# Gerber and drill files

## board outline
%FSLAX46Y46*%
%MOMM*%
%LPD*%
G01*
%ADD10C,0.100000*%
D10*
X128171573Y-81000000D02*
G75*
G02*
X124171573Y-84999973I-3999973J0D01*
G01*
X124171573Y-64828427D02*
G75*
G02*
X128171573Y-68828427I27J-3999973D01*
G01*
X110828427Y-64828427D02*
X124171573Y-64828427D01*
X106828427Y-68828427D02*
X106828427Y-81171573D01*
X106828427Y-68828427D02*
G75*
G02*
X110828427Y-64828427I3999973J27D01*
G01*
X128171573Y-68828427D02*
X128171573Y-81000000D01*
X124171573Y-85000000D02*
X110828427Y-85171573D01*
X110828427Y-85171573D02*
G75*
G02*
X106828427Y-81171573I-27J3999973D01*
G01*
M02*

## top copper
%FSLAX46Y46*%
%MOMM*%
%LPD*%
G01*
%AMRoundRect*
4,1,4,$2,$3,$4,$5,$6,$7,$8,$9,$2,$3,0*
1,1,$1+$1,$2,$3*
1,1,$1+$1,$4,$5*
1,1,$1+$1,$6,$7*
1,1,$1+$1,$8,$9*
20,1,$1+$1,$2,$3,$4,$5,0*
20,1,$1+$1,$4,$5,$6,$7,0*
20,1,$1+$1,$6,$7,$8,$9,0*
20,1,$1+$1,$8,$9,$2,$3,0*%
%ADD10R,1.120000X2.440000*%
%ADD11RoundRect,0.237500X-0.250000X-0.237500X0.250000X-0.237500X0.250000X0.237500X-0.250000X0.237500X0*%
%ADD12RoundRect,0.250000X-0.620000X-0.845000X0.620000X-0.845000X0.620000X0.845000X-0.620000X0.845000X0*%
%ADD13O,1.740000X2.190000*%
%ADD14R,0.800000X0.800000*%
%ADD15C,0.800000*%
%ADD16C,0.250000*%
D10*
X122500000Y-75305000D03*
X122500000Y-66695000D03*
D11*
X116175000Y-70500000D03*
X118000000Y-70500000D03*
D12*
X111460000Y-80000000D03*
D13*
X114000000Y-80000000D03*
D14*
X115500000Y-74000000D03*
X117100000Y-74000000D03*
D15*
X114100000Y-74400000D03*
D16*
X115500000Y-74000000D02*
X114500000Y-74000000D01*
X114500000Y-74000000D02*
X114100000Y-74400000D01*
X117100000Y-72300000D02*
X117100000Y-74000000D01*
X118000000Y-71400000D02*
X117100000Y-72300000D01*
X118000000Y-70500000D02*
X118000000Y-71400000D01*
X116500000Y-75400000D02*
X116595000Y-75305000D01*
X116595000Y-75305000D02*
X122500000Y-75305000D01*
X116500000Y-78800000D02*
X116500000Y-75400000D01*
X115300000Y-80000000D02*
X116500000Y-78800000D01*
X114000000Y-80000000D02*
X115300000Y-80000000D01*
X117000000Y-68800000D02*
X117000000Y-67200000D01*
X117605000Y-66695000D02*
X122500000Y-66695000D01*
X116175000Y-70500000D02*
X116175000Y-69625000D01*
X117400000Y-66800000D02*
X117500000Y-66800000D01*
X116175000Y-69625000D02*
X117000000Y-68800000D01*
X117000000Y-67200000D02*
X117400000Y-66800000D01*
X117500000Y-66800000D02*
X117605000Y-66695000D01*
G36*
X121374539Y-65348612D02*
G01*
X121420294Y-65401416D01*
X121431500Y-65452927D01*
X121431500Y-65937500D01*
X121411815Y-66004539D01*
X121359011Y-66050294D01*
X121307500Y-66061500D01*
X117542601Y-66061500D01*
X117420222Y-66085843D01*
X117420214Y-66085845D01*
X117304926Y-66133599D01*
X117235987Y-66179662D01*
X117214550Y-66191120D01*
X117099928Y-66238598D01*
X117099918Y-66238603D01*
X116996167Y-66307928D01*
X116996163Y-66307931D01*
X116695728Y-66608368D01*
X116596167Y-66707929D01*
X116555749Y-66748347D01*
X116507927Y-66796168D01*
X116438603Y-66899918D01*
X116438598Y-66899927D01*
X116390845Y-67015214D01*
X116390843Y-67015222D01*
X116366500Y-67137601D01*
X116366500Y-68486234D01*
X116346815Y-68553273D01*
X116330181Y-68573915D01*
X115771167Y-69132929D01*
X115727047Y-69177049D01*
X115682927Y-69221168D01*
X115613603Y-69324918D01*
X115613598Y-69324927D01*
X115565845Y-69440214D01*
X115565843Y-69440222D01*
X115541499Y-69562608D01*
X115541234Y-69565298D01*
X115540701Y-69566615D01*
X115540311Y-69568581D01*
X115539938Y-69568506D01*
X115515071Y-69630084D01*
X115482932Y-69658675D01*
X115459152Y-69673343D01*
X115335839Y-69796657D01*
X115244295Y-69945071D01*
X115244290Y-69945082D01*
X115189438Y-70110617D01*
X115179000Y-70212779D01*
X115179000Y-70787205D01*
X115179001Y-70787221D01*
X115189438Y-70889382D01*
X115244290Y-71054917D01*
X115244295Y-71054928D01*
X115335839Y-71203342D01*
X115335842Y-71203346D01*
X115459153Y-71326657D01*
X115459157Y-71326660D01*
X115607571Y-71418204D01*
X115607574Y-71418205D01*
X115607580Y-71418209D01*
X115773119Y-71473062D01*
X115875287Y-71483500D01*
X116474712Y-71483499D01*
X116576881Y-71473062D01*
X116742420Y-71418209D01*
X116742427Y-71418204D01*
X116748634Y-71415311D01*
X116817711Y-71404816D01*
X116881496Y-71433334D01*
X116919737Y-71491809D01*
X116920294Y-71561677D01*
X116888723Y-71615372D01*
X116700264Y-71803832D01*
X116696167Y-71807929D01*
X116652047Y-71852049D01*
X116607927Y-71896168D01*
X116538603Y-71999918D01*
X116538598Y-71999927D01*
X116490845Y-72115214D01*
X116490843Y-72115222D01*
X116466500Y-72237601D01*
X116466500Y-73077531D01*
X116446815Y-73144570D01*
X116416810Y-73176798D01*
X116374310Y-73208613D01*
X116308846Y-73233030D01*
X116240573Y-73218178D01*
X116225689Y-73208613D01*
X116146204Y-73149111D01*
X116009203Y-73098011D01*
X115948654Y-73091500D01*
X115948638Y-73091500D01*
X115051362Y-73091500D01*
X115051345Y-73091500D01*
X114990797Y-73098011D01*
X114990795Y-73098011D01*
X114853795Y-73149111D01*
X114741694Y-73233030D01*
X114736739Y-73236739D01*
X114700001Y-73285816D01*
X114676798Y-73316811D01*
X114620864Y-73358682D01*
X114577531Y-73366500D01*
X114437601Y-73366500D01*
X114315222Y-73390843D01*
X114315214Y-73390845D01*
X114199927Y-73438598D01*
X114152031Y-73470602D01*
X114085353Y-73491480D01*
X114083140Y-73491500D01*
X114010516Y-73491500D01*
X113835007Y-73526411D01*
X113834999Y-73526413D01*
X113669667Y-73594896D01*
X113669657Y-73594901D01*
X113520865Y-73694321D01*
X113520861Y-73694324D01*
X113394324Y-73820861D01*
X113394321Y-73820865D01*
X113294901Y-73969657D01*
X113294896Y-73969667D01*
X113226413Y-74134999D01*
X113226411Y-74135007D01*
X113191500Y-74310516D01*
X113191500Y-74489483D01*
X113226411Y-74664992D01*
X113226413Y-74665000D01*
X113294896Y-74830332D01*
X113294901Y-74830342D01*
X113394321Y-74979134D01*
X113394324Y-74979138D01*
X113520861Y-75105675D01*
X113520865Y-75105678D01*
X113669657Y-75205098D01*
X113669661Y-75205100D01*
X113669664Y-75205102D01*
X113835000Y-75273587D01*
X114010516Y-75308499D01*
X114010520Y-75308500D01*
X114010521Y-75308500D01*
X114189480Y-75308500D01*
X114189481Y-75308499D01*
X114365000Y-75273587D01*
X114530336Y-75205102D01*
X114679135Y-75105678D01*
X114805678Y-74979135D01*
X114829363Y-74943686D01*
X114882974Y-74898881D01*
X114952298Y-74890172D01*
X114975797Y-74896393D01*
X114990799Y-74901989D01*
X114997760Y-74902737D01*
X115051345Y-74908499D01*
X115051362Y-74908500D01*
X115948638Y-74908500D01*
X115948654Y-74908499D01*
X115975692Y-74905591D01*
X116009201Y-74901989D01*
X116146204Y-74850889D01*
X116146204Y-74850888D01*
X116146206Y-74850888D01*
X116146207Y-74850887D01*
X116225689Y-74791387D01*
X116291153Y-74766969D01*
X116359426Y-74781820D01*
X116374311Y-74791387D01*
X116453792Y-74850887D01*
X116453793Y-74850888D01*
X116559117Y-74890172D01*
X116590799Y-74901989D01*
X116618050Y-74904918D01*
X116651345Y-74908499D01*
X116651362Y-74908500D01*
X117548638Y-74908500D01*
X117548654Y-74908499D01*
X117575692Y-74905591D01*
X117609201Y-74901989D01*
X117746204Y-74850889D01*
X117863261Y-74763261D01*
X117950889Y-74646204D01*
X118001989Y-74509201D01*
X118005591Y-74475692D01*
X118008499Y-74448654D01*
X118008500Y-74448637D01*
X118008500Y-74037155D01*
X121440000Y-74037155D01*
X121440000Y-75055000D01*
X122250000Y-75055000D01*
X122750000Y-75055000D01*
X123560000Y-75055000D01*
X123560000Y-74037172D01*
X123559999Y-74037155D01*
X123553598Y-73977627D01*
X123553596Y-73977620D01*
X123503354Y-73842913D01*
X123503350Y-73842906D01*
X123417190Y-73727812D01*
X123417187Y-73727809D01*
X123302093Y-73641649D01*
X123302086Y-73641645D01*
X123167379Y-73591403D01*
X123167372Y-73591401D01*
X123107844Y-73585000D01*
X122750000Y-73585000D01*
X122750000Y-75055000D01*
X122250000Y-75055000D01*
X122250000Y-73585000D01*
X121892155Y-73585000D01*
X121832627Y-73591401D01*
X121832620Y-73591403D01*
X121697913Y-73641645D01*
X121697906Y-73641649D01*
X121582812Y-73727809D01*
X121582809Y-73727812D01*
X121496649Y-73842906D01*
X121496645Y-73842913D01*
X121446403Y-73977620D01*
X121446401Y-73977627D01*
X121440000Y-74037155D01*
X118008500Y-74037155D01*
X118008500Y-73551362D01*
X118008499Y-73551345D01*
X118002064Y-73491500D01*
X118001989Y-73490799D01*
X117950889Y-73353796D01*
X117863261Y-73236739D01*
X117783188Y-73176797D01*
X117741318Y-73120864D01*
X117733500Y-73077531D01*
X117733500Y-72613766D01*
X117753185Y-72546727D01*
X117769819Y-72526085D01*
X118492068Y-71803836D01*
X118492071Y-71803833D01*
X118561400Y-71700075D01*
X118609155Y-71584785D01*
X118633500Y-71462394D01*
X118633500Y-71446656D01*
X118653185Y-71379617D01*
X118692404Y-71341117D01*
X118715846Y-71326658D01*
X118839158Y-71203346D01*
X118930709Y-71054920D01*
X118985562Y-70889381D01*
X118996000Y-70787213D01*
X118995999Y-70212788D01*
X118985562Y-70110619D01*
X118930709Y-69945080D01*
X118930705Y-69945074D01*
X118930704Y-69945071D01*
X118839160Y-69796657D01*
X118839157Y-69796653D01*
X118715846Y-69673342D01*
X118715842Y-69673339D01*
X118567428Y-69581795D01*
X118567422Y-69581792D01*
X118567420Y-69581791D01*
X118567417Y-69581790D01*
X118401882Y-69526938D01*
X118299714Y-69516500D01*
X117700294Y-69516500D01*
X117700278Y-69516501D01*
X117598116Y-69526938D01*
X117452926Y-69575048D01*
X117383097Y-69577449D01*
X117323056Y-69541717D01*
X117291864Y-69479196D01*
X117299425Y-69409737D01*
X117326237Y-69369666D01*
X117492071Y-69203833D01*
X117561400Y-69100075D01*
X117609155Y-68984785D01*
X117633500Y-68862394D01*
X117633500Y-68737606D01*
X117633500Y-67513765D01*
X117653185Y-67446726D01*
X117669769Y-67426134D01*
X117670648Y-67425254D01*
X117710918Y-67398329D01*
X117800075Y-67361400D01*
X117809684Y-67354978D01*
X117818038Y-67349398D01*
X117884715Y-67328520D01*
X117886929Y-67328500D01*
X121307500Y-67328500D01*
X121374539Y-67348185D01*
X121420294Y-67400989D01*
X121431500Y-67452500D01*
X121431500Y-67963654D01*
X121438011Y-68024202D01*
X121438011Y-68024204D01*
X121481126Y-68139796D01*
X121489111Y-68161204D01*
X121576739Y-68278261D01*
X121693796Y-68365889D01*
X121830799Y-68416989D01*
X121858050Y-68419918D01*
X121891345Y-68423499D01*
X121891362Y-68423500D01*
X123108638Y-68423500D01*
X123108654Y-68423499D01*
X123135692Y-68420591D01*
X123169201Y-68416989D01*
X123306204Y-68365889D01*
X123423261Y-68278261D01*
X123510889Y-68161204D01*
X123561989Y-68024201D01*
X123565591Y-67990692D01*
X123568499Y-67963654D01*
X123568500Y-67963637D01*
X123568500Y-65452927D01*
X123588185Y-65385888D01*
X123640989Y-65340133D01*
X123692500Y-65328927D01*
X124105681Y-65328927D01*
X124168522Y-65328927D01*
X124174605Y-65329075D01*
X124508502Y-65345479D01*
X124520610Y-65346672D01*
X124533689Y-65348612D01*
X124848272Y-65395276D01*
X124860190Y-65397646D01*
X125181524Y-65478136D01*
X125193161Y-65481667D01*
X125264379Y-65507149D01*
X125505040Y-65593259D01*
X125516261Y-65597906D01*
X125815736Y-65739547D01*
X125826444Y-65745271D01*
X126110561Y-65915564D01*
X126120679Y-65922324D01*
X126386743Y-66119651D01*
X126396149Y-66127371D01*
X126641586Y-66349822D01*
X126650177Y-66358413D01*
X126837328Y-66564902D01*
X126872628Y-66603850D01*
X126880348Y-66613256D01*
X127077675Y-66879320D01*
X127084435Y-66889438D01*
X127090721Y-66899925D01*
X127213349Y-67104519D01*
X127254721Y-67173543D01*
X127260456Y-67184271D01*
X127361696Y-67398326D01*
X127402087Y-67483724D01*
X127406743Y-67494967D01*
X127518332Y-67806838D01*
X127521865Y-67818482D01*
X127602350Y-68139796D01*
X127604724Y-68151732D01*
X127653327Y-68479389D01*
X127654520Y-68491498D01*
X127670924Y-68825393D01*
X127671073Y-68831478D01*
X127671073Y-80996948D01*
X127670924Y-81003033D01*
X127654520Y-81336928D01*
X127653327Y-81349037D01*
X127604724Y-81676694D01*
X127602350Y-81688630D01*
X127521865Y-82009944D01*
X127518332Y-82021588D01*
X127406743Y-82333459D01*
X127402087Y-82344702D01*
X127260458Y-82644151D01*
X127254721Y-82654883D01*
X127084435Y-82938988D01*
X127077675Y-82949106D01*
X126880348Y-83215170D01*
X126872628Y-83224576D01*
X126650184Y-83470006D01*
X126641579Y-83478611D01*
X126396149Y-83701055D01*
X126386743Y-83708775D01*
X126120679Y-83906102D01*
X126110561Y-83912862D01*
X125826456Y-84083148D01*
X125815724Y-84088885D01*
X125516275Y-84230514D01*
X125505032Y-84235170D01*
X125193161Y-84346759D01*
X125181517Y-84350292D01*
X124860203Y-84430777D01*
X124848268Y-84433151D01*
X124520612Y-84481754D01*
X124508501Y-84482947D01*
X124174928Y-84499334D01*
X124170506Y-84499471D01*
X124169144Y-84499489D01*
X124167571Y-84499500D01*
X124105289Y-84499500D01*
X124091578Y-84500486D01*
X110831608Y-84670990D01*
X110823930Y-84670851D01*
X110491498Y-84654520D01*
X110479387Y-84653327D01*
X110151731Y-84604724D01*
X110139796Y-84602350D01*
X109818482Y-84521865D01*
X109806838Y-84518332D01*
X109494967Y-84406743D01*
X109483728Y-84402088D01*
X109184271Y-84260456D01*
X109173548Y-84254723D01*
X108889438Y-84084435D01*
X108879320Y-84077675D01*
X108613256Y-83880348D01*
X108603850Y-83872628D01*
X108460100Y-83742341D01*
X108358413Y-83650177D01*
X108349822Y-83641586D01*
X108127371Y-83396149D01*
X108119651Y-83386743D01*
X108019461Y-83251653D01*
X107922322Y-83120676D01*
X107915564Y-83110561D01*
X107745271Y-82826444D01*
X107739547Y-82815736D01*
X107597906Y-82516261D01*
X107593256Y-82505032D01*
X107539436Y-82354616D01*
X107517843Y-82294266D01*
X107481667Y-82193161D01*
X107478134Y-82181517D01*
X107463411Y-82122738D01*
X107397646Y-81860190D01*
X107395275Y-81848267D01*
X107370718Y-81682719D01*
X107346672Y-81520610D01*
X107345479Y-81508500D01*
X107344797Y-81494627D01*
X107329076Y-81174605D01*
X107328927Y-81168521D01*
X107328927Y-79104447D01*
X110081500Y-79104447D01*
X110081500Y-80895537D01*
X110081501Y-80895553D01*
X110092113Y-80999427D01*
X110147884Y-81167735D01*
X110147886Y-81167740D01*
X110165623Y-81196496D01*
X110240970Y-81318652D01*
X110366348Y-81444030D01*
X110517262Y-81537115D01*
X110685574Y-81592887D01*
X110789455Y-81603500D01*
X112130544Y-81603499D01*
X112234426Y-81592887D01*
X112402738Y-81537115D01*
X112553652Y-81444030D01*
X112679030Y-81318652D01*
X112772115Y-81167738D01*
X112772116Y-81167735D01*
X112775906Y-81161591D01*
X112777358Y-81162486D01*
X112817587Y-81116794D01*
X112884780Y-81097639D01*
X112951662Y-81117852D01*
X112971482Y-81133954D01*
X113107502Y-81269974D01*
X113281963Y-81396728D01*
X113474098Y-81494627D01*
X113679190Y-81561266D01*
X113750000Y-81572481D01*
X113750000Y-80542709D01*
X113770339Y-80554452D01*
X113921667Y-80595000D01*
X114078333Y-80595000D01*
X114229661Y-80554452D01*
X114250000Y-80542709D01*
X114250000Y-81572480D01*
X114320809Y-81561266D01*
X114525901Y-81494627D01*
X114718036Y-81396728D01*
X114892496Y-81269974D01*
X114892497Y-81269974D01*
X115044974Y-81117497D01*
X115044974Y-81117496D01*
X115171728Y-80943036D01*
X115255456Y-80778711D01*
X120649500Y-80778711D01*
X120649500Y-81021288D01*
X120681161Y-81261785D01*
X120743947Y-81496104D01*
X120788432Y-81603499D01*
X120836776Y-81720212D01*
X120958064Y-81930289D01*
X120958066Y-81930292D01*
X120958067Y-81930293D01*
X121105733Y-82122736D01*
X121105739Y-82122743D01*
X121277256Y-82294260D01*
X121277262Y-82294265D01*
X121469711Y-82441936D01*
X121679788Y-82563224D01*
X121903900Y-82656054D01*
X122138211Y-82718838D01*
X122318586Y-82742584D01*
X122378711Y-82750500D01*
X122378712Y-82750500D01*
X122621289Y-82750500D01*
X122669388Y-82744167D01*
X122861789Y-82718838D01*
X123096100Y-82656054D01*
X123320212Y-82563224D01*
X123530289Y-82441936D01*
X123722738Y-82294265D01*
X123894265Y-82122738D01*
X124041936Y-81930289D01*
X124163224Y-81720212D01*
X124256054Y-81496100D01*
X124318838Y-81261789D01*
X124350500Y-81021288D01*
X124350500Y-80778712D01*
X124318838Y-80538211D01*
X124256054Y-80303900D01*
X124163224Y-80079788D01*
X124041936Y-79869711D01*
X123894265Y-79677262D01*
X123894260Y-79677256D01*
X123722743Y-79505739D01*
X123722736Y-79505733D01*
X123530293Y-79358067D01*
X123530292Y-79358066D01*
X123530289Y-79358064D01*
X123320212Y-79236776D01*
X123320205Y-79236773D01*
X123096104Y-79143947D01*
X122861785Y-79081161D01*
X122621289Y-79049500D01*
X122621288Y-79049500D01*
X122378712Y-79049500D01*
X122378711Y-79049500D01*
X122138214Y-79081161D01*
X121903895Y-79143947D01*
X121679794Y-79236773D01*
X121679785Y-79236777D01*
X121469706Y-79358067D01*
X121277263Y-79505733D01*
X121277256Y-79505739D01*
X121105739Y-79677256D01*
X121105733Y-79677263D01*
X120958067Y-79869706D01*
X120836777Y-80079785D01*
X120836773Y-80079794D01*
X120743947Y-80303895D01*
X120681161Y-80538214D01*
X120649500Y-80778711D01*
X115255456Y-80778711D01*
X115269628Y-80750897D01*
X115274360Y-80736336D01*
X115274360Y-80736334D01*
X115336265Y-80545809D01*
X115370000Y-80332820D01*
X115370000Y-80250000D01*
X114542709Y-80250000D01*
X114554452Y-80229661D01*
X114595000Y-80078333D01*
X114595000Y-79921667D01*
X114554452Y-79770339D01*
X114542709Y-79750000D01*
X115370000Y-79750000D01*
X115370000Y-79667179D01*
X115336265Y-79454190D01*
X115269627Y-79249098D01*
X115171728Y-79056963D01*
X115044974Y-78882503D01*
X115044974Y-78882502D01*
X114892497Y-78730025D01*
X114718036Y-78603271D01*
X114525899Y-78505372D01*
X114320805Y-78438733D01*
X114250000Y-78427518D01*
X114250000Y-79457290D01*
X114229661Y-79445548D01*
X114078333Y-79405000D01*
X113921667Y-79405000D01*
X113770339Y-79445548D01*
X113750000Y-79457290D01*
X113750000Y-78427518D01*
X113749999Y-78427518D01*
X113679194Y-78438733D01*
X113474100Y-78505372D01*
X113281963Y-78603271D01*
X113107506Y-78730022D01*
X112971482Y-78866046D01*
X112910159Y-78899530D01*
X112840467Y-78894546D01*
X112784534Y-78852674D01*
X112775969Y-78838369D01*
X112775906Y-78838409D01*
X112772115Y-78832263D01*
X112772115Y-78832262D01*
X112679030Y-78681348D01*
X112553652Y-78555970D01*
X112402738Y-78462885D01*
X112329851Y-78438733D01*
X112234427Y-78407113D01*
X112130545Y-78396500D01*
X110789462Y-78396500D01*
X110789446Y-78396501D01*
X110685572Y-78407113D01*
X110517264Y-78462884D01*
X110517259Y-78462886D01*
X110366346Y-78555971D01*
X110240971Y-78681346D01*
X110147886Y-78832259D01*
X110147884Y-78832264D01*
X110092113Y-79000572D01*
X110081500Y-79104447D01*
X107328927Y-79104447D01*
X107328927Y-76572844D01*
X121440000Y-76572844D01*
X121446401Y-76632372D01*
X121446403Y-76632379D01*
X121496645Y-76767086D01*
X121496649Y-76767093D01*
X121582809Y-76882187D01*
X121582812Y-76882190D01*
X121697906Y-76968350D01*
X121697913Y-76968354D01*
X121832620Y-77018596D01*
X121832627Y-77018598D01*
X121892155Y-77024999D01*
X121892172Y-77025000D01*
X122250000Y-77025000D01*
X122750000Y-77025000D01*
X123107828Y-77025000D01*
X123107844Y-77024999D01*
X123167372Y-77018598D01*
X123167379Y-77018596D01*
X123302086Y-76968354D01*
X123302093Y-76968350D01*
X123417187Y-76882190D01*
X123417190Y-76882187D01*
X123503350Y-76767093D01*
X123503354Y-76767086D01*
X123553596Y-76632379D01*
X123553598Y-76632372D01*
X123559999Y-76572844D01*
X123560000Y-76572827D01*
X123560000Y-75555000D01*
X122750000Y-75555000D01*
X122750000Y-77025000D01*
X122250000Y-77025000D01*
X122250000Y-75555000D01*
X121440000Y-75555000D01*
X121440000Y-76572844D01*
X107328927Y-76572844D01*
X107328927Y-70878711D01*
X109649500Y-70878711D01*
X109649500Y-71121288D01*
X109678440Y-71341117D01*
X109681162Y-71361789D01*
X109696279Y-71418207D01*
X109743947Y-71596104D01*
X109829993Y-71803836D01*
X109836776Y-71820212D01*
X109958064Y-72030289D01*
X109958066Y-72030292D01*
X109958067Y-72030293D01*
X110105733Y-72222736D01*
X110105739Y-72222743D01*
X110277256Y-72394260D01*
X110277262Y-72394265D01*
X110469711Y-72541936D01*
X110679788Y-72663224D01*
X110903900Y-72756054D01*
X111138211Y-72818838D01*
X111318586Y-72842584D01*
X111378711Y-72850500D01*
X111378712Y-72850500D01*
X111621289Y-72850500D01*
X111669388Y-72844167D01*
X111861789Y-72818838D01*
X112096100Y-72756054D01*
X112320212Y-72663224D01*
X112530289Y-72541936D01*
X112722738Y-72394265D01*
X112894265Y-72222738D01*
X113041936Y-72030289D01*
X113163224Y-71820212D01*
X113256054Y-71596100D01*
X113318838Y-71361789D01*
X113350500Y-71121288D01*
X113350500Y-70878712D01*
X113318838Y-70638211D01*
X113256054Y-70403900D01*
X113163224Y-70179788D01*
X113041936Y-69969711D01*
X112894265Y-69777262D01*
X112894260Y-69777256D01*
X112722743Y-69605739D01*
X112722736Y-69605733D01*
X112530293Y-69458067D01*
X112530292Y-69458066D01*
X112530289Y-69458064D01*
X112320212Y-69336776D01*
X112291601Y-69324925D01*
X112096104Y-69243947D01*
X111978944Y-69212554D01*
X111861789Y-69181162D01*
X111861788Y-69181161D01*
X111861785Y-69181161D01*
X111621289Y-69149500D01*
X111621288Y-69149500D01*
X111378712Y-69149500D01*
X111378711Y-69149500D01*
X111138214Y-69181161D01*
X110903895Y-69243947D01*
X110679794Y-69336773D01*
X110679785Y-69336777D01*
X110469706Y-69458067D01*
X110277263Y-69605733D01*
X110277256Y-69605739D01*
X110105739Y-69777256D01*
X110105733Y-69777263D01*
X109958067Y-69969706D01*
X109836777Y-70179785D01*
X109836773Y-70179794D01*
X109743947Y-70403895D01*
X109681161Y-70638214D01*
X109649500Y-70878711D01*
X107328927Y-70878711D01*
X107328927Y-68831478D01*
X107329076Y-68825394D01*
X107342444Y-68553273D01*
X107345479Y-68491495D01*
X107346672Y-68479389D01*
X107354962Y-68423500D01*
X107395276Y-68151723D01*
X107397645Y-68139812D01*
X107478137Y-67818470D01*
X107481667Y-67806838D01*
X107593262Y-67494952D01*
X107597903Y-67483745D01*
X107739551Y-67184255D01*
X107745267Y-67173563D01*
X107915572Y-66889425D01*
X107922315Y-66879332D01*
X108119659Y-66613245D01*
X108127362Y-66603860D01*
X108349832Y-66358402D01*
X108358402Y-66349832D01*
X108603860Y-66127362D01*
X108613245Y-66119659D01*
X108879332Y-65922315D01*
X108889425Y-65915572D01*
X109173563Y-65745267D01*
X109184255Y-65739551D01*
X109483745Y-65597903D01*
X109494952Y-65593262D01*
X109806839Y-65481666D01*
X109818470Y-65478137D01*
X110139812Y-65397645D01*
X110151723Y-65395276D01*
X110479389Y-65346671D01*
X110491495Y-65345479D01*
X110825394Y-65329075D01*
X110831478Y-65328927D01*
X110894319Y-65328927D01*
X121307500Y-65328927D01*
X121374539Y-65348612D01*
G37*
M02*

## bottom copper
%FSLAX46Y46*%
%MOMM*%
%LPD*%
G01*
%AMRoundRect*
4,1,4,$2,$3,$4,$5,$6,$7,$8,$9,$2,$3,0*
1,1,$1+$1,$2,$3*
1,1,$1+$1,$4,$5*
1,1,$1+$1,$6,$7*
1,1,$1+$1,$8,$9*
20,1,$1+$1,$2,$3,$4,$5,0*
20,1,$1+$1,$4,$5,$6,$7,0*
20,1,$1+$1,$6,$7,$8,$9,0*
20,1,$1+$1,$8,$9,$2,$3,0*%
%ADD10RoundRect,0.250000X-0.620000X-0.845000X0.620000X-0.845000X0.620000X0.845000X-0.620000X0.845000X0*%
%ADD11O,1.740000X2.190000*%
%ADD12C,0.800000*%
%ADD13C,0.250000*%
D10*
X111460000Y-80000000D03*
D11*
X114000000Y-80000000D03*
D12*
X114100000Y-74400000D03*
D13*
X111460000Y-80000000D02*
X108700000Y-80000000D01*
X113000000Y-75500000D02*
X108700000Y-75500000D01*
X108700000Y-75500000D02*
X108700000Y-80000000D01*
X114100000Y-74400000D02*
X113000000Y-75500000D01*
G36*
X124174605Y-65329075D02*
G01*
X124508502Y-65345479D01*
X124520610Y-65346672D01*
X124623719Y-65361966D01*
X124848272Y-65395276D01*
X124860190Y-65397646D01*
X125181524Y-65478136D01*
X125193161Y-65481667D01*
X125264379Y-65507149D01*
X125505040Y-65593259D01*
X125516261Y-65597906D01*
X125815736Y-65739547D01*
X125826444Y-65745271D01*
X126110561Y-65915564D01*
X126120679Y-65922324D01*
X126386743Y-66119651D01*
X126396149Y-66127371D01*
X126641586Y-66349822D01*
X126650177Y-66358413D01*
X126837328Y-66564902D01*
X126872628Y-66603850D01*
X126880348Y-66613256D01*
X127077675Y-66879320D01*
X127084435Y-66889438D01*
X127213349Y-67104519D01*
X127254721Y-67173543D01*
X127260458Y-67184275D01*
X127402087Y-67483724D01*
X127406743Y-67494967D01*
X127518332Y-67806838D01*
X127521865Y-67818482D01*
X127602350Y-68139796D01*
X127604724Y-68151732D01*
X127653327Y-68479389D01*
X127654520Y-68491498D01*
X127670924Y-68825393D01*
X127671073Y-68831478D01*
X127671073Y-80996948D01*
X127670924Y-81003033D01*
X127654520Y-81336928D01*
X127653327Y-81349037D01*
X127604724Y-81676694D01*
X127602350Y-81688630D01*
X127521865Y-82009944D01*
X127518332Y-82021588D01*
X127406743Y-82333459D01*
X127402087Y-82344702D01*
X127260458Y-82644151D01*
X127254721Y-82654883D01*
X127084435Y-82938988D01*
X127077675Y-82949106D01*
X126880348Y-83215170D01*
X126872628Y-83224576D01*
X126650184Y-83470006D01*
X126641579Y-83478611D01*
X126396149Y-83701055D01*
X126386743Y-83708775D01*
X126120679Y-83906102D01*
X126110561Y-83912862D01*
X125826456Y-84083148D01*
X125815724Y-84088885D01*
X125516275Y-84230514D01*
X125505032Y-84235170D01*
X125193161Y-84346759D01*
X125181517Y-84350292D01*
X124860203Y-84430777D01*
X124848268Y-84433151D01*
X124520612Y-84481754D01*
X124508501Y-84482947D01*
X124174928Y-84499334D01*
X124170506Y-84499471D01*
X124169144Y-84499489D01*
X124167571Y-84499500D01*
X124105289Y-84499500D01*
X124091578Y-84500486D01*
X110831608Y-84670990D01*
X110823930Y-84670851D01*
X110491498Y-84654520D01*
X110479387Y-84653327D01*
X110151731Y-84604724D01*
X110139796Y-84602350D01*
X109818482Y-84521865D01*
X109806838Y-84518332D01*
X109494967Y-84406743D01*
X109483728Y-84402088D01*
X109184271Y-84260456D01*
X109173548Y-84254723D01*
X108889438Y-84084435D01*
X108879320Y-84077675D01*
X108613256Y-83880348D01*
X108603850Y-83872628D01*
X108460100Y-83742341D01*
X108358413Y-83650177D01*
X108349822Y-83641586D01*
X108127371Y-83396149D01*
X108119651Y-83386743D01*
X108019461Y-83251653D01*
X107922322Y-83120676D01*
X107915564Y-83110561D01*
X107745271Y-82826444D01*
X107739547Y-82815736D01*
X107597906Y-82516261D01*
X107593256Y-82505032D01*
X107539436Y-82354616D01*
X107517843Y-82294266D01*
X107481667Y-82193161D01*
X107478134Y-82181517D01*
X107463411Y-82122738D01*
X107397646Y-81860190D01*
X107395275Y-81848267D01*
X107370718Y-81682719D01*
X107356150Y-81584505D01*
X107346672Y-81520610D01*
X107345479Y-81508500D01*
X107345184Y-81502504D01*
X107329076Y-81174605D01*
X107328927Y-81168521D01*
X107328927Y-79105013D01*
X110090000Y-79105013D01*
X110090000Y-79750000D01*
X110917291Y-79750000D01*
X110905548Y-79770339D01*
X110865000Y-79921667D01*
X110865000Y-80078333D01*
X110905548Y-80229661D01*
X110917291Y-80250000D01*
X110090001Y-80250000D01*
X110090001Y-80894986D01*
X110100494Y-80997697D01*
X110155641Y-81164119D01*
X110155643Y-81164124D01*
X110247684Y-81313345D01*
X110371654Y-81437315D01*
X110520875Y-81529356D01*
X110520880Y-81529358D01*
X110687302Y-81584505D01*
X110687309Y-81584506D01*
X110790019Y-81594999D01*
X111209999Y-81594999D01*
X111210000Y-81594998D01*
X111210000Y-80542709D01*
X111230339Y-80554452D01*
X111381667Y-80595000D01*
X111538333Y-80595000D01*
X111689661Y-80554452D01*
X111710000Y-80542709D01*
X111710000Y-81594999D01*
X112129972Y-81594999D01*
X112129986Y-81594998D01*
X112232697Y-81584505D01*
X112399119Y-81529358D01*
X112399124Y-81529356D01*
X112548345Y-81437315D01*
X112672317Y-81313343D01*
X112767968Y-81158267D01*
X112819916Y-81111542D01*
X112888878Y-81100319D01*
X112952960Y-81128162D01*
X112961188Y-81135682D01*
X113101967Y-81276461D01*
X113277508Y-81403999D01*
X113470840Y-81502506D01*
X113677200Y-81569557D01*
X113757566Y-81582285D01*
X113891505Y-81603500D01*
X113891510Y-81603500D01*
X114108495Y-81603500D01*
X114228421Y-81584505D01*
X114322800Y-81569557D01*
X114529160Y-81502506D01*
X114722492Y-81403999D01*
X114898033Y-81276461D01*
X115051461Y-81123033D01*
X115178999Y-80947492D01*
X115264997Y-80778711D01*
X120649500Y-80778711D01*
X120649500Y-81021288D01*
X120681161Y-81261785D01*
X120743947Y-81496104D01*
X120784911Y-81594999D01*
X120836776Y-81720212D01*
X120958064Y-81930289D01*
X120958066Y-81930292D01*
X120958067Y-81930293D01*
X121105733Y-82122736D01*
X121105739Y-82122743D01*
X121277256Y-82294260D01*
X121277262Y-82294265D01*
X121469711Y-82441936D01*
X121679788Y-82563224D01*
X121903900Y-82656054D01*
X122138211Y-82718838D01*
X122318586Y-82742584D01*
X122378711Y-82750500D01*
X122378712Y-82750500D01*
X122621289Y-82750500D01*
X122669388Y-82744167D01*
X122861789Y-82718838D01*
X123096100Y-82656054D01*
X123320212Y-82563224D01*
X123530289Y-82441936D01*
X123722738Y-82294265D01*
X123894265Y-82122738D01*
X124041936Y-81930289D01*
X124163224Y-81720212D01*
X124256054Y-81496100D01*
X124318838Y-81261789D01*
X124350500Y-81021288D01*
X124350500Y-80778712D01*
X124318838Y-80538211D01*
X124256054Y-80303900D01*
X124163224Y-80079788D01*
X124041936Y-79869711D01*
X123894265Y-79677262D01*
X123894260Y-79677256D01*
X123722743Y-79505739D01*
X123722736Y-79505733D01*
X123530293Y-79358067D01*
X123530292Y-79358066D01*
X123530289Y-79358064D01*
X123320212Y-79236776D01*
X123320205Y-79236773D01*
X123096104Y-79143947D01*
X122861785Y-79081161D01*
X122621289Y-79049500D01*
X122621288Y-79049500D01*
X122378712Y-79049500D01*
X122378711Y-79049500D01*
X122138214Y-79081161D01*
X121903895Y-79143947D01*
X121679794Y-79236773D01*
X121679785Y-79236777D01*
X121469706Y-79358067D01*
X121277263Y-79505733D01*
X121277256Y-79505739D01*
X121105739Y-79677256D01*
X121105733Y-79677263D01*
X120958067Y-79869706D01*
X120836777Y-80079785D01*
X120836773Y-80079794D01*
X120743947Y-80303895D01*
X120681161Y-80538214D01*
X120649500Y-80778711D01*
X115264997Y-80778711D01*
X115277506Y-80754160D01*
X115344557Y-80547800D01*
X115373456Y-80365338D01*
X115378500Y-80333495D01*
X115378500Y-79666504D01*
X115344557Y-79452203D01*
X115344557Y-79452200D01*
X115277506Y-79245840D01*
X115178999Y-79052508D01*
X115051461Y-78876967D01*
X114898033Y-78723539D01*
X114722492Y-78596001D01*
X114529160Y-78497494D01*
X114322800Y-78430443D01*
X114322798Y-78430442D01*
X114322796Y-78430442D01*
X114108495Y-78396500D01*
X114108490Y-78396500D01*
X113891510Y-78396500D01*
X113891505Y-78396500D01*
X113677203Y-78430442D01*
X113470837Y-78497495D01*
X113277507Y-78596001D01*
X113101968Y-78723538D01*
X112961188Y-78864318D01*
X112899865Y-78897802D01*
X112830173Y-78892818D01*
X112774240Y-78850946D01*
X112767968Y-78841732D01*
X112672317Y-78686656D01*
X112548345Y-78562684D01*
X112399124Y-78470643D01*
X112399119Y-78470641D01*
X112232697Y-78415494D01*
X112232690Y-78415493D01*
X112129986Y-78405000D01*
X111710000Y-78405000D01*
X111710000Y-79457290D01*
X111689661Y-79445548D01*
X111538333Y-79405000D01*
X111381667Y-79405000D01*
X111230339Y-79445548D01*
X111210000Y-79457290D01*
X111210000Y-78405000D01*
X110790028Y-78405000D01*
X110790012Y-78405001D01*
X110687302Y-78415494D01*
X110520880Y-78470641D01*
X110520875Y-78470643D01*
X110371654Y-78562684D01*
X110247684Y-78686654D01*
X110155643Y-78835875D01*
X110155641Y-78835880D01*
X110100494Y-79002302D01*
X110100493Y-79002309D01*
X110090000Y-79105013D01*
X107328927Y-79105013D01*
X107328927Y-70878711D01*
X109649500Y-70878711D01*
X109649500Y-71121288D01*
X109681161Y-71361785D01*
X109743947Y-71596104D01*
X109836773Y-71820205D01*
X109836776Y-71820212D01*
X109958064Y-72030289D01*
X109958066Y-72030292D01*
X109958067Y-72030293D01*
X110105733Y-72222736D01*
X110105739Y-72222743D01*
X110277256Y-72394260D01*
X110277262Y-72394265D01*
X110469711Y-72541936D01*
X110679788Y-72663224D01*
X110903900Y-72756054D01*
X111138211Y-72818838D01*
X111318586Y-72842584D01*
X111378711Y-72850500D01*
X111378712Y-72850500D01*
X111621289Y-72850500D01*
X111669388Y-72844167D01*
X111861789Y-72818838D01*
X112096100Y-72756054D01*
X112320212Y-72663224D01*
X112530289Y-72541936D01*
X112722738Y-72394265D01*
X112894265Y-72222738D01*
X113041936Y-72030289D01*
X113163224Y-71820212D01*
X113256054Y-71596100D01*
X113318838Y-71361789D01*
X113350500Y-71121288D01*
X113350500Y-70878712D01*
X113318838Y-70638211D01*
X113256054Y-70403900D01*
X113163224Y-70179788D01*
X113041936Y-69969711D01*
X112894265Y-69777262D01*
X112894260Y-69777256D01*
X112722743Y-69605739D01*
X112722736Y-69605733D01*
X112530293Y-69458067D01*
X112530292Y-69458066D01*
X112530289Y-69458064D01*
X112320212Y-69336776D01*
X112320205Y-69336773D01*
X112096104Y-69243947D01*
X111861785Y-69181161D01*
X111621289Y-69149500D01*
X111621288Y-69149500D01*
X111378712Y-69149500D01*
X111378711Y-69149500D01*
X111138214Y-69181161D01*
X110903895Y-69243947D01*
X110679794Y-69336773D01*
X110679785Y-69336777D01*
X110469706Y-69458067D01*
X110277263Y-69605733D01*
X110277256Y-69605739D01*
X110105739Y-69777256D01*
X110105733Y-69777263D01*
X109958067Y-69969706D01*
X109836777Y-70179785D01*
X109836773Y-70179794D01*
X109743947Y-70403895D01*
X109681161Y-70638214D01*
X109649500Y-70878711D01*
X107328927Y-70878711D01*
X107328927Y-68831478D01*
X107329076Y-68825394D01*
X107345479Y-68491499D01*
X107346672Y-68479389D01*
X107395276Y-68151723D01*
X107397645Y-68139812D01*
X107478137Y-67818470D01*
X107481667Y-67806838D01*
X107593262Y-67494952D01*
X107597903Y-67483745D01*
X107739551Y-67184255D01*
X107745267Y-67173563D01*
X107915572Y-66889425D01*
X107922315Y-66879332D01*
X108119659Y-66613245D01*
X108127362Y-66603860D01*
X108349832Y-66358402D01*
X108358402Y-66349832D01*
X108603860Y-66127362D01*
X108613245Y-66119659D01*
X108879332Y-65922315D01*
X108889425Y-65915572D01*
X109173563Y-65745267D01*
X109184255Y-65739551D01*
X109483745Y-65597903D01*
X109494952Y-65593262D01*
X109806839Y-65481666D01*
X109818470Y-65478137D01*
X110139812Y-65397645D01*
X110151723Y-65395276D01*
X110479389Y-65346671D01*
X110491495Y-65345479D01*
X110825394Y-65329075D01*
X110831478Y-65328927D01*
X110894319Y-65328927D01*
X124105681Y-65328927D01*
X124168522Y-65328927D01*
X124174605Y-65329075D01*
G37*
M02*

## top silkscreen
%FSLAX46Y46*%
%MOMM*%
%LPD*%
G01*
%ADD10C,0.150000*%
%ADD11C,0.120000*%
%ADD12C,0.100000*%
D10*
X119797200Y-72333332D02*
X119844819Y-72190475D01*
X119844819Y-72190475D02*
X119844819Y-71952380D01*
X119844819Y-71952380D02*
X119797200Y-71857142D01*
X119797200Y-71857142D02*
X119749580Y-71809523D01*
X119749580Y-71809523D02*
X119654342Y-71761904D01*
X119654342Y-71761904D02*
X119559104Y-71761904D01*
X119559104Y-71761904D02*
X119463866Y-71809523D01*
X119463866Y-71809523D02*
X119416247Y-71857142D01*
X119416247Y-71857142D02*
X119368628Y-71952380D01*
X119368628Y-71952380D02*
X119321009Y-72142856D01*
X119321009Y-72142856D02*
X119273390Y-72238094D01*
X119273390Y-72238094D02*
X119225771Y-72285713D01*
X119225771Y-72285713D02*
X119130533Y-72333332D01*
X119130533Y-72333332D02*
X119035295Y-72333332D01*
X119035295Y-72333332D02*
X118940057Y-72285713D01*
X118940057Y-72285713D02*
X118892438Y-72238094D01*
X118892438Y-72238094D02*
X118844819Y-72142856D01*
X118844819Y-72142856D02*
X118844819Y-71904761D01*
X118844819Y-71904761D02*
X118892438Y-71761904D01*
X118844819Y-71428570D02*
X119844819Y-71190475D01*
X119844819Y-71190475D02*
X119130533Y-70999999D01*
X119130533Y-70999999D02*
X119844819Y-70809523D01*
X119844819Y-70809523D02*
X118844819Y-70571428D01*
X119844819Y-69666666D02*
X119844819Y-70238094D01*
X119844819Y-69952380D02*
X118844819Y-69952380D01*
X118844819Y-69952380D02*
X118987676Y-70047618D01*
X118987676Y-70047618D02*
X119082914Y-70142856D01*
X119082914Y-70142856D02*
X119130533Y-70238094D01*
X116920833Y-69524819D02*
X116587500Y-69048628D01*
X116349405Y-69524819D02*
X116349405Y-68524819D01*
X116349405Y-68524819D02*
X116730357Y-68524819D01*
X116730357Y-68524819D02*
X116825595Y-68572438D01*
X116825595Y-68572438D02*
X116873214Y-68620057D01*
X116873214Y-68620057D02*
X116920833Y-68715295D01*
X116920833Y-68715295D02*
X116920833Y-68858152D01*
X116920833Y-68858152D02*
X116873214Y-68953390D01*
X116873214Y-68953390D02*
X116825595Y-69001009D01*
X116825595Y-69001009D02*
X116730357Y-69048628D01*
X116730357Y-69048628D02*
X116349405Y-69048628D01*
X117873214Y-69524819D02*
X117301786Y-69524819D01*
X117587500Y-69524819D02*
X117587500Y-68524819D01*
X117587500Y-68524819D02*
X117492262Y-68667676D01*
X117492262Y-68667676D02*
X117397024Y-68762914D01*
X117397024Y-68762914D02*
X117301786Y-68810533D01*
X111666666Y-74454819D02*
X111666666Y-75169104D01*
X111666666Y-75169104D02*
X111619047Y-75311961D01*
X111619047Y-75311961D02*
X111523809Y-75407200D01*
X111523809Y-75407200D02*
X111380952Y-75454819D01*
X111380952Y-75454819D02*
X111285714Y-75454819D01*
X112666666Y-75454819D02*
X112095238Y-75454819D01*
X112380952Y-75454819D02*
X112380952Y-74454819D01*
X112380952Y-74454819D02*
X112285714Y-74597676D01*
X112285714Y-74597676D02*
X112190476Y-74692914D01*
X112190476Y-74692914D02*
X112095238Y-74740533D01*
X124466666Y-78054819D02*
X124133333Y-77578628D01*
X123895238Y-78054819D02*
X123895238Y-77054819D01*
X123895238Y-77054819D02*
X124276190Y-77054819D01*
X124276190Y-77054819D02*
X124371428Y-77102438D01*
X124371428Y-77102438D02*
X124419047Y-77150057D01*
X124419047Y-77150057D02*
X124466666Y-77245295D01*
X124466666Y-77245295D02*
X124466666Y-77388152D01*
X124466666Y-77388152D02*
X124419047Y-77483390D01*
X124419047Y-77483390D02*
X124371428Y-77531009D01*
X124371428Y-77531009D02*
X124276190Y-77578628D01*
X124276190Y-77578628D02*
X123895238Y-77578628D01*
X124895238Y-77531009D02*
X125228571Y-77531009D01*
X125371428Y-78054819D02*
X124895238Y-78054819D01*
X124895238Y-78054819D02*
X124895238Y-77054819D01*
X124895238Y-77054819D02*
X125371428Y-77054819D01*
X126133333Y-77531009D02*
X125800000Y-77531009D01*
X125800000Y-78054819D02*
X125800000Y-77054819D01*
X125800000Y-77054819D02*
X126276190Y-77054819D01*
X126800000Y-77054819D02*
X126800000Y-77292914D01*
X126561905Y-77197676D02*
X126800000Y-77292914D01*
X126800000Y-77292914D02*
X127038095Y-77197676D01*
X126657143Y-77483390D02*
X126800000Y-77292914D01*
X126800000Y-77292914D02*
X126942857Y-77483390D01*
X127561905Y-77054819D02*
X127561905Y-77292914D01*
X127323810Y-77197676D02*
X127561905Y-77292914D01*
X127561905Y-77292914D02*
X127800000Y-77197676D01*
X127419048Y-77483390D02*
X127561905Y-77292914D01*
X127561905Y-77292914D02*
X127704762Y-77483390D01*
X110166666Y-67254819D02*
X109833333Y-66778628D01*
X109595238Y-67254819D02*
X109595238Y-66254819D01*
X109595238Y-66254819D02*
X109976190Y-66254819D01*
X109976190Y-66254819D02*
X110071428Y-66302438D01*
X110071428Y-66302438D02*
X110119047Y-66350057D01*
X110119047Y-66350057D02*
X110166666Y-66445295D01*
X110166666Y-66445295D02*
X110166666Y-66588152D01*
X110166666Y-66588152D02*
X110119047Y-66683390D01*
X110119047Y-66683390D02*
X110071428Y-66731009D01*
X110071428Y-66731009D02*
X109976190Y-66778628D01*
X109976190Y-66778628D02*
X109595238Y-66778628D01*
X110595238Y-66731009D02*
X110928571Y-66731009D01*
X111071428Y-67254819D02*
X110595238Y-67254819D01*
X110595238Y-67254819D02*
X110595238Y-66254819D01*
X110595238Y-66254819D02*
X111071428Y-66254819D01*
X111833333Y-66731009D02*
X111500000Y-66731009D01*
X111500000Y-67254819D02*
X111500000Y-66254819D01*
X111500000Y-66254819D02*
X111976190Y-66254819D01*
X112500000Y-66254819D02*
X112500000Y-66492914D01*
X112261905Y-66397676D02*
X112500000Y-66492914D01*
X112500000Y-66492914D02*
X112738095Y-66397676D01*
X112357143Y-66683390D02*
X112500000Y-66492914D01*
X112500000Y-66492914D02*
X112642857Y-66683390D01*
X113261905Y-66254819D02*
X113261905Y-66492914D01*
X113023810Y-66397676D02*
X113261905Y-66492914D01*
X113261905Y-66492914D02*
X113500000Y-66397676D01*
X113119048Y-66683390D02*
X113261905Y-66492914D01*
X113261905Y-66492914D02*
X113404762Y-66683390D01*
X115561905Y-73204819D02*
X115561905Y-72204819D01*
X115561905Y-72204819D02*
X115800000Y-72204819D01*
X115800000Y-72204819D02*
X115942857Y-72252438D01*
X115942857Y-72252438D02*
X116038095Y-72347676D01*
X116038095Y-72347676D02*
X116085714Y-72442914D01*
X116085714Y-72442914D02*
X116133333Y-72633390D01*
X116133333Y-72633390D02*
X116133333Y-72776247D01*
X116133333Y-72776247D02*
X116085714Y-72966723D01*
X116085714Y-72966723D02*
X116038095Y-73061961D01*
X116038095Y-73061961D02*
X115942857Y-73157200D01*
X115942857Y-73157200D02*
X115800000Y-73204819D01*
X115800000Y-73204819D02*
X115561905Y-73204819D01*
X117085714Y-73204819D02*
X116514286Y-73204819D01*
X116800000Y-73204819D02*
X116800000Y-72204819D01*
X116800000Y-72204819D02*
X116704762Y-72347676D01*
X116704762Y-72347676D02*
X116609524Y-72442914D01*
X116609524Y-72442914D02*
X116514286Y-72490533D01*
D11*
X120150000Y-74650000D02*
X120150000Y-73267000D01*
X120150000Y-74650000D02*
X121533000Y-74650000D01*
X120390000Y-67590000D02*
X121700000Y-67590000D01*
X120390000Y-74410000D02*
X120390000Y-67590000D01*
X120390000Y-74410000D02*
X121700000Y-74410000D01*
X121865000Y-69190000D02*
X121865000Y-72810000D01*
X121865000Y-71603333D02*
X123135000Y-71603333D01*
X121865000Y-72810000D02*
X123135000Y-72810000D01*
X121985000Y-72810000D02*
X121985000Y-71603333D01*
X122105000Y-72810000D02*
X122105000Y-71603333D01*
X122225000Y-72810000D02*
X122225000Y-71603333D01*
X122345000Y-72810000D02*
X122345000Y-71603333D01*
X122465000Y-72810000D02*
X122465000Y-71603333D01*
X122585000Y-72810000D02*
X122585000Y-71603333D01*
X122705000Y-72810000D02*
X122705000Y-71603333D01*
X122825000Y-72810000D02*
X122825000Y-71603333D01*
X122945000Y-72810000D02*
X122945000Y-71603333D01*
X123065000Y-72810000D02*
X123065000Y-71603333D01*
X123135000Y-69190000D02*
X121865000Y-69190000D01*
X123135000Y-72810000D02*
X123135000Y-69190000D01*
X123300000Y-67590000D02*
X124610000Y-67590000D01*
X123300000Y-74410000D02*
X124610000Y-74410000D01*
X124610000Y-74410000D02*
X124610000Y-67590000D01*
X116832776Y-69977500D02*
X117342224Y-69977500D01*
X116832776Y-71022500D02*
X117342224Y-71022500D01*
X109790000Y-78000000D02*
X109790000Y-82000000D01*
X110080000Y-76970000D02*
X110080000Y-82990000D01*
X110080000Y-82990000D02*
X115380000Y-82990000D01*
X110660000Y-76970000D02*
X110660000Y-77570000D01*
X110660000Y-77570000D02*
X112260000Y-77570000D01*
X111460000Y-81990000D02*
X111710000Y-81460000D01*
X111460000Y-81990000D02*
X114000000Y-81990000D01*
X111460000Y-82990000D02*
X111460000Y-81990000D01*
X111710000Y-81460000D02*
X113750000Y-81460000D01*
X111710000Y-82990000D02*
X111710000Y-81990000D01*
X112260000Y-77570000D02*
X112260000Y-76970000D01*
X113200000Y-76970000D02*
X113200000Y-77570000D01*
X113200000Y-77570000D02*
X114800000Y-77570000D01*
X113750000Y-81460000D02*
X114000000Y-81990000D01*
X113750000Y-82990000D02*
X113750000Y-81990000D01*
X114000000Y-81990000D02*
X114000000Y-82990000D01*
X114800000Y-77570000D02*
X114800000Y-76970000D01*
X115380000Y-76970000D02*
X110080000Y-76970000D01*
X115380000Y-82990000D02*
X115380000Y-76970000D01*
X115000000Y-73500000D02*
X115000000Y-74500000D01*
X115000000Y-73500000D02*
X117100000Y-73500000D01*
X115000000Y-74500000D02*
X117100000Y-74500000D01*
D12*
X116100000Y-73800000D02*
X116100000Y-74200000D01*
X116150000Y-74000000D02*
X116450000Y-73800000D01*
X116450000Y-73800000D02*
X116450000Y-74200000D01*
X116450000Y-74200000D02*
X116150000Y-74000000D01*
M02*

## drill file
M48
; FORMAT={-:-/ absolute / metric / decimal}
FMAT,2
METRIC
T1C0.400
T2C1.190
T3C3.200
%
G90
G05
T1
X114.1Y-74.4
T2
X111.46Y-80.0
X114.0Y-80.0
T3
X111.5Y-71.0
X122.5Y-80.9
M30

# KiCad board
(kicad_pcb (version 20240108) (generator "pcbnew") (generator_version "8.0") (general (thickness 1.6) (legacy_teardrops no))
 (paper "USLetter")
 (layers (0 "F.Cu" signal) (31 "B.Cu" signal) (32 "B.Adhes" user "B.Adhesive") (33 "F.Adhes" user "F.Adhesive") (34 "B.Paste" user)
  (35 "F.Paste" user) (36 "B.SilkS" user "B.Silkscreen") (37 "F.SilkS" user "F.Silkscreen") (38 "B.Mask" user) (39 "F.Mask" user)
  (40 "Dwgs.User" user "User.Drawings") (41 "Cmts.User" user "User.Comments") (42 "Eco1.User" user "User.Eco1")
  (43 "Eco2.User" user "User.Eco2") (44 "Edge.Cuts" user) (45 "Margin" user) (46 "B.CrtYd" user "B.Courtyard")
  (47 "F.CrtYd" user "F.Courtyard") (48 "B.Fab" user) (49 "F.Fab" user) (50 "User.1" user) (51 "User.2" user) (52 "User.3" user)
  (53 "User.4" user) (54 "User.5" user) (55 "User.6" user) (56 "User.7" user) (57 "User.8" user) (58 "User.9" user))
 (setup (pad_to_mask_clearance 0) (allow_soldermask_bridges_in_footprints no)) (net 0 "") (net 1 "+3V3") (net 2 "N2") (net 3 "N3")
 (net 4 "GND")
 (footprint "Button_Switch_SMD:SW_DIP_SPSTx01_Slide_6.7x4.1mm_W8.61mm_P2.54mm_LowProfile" (layer "F.Cu") (at 122.5 71 90)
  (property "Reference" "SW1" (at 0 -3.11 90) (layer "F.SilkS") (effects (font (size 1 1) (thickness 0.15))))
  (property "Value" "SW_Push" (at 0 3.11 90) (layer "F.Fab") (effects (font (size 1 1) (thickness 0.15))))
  (fp_line (start -3.65 -2.35) (end -2.267 -2.35) (stroke (width 0.12) (type solid)) (layer "F.SilkS"))
  (fp_line (start -3.65 -2.35) (end -3.65 -0.967) (stroke (width 0.12) (type solid)) (layer "F.SilkS"))
  (fp_line (start 3.41 -2.11) (end 3.41 -0.8) (stroke (width 0.12) (type solid)) (layer "F.SilkS"))
  (fp_line (start -3.41 -2.11) (end 3.41 -2.11) (stroke (width 0.12) (type solid)) (layer "F.SilkS"))
  (fp_line (start -3.41 -2.11) (end -3.41 -0.8) (stroke (width 0.12) (type solid)) (layer "F.SilkS"))
  (fp_line (start 1.81 -0.635) (end -1.81 -0.635) (stroke (width 0.12) (type solid)) (layer "F.SilkS"))
  (fp_line (start -0.603333 -0.635) (end -0.603333 0.635) (stroke (width 0.12) (type solid)) (layer "F.SilkS"))
  (fp_line (start -1.81 -0.635) (end -1.81 0.635) (stroke (width 0.12) (type solid)) (layer "F.SilkS"))
  (fp_line (start -1.81 -0.515) (end -0.603333 -0.515) (stroke (width 0.12) (type solid)) (layer "F.SilkS"))
  (fp_line (start -1.81 -0.395) (end -0.603333 -0.395) (stroke (width 0.12) (type solid)) (layer "F.SilkS"))
  (fp_line (start -1.81 -0.275) (end -0.603333 -0.275) (stroke (width 0.12) (type solid)) (layer "F.SilkS"))
  (fp_line (start -1.81 -0.155) (end -0.603333 -0.155) (stroke (width 0.12) (type solid)) (layer "F.SilkS"))
  (fp_line (start -1.81 -0.035) (end -0.603333 -0.035) (stroke (width 0.12) (type solid)) (layer "F.SilkS"))
  (fp_line (start -1.81 0.085) (end -0.603333 0.085) (stroke (width 0.12) (type solid)) (layer "F.SilkS"))
  (fp_line (start -1.81 0.205) (end -0.603333 0.205) (stroke (width 0.12) (type solid)) (layer "F.SilkS"))
  (fp_line (start -1.81 0.325) (end -0.603333 0.325) (stroke (width 0.12) (type solid)) (layer "F.SilkS"))
  (fp_line (start -1.81 0.445) (end -0.603333 0.445) (stroke (width 0.12) (type solid)) (layer "F.SilkS"))
  (fp_line (start -1.81 0.565) (end -0.603333 0.565) (stroke (width 0.12) (type solid)) (layer "F.SilkS"))
  (fp_line (start 1.81 0.635) (end 1.81 -0.635) (stroke (width 0.12) (type solid)) (layer "F.SilkS"))
  (fp_line (start -1.81 0.635) (end 1.81 0.635) (stroke (width 0.12) (type solid)) (layer "F.SilkS"))
  (fp_line (start 3.41 0.8) (end 3.41 2.11) (stroke (width 0.12) (type solid)) (layer "F.SilkS"))
  (fp_line (start -3.41 0.8) (end -3.41 2.11) (stroke (width 0.12) (type solid)) (layer "F.SilkS"))
  (fp_line (start -3.41 2.11) (end 3.41 2.11) (stroke (width 0.12) (type solid)) (layer "F.SilkS"))
  (pad "1" smd rect (at -4.305 0 90) (size 2.44 1.12) (layers "F.Cu" "F.Paste" "F.Mask") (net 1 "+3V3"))
  (pad "2" smd rect (at 4.305 0 90) (size 2.44 1.12) (layers "F.Cu" "F.Paste" "F.Mask") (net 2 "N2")))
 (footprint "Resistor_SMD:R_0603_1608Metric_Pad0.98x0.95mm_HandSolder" (layer "F.Cu") (at 117.0875 70.5)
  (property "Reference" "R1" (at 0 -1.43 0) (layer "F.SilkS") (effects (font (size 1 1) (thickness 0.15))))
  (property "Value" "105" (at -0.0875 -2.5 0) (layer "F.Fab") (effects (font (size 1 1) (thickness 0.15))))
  (fp_line (start -0.254724 -0.5225) (end 0.254724 -0.5225) (stroke (width 0.12) (type solid)) (layer "F.SilkS"))
  (fp_line (start -0.254724 0.5225) (end 0.254724 0.5225) (stroke (width 0.12) (type solid)) (layer "F.SilkS"))
  (pad "1" smd roundrect (at -0.9125 0) (size 0.975 0.95) (layers "F.Cu" "F.Paste" "F.Mask") (roundrect_rratio 0.25) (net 2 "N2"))
  (pad "2" smd roundrect (at 0.9125 0) (size 0.975 0.95) (layers "F.Cu" "F.Paste" "F.Mask") (roundrect_rratio 0.25) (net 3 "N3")))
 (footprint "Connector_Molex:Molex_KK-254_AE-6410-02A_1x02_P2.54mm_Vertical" (layer "F.Cu") (at 111.46 80)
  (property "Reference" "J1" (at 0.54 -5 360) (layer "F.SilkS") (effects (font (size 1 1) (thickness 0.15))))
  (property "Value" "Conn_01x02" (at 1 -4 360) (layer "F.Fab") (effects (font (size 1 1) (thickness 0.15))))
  (fp_line (start -1.67 -2) (end -1.67 2) (stroke (width 0.12) (type solid)) (layer "F.SilkS"))
  (fp_line (start -1.38 -3.03) (end -1.38 2.99) (stroke (width 0.12) (type solid)) (layer "F.SilkS"))
  (fp_line (start -1.38 2.99) (end 3.92 2.99) (stroke (width 0.12) (type solid)) (layer "F.SilkS"))
  (fp_line (start -0.8 -3.03) (end -0.8 -2.43) (stroke (width 0.12) (type solid)) (layer "F.SilkS"))
  (fp_line (start -0.8 -2.43) (end 0.8 -2.43) (stroke (width 0.12) (type solid)) (layer "F.SilkS"))
  (fp_line (start 0 1.99) (end 0.25 1.46) (stroke (width 0.12) (type solid)) (layer "F.SilkS"))
  (fp_line (start 0 1.99) (end 2.54 1.99) (stroke (width 0.12) (type solid)) (layer "F.SilkS"))
  (fp_line (start 0 2.99) (end 0 1.99) (stroke (width 0.12) (type solid)) (layer "F.SilkS"))
  (fp_line (start 0.25 1.46) (end 2.29 1.46) (stroke (width 0.12) (type solid)) (layer "F.SilkS"))
  (fp_line (start 0.25 2.99) (end 0.25 1.99) (stroke (width 0.12) (type solid)) (layer "F.SilkS"))
  (fp_line (start 0.8 -2.43) (end 0.8 -3.03) (stroke (width 0.12) (type solid)) (layer "F.SilkS"))
  (fp_line (start 1.74 -3.03) (end 1.74 -2.43) (stroke (width 0.12) (type solid)) (layer "F.SilkS"))
  (fp_line (start 1.74 -2.43) (end 3.34 -2.43) (stroke (width 0.12) (type solid)) (layer "F.SilkS"))
  (fp_line (start 2.29 1.46) (end 2.54 1.99) (stroke (width 0.12) (type solid)) (layer "F.SilkS"))
  (fp_line (start 2.29 2.99) (end 2.29 1.99) (stroke (width 0.12) (type solid)) (layer "F.SilkS"))
  (fp_line (start 2.54 1.99) (end 2.54 2.99) (stroke (width 0.12) (type solid)) (layer "F.SilkS"))
  (fp_line (start 3.34 -2.43) (end 3.34 -3.03) (stroke (width 0.12) (type solid)) (layer "F.SilkS"))
  (fp_line (start 3.92 -3.03) (end -1.38 -3.03) (stroke (width 0.12) (type solid)) (layer "F.SilkS"))
  (fp_line (start 3.92 2.99) (end 3.92 -3.03) (stroke (width 0.12) (type solid)) (layer "F.SilkS"))
  (pad "1" thru_hole roundrect (at 0 0) (size 1.74 2.19) (drill 1.19) (layers "*.Cu" "*.Mask") (remove_unused_layers no)
   (roundrect_rratio 0.143678) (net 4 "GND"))
  (pad "2" thru_hole oval (at 2.54 0) (size 1.74 2.19) (drill 1.19) (layers "*.Cu" "*.Mask") (remove_unused_layers no) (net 1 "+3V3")))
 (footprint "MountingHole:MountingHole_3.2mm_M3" (layer "F.Cu") (at 122.5 80.9)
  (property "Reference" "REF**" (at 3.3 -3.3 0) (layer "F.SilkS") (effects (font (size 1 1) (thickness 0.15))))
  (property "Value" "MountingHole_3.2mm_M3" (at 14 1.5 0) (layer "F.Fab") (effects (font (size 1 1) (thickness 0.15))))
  (pad "" np_thru_hole circle (at 0 0) (size 3.2 3.2) (drill 3.2) (layers "*.Cu" "*.Mask")))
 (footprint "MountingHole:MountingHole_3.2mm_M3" (layer "F.Cu") (at 111.5 71)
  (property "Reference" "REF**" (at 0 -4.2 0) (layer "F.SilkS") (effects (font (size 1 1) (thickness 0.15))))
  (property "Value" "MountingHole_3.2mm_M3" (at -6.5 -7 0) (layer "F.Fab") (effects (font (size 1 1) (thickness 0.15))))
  (pad "" np_thru_hole circle (at 0 0) (size 3.2 3.2) (drill 3.2) (layers "*.Cu" "*.Mask")))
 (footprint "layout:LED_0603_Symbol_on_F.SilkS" (layer "F.Cu") (at 116.3 74)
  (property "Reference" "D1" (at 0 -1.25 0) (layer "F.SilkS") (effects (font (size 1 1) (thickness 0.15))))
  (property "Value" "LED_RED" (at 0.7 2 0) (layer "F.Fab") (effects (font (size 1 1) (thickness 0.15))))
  (fp_line (start -1.3 -0.5) (end -1.3 0.5) (stroke (width 0.12) (type solid)) (layer "F.SilkS"))
  (fp_line (start -1.3 -0.5) (end 0.8 -0.5) (stroke (width 0.12) (type solid)) (layer "F.SilkS"))
  (fp_line (start -1.3 0.5) (end 0.8 0.5) (stroke (width 0.12) (type solid)) (layer "F.SilkS"))
  (fp_line (start -0.2 -0.2) (end -0.2 0.2) (stroke (width 0.1) (type solid)) (layer "F.SilkS"))
  (fp_line (start -0.15 0) (end 0.15 -0.2) (stroke (width 0.1) (type solid)) (layer "F.SilkS"))
  (fp_line (start 0.15 -0.2) (end 0.15 0.2) (stroke (width 0.1) (type solid)) (layer "F.SilkS"))
  (fp_line (start 0.15 0.2) (end -0.15 0) (stroke (width 0.1) (type solid)) (layer "F.SilkS"))
  (pad "1" smd rect (at -0.8 0 180) (size 0.8 0.8) (layers "F.Cu" "F.Paste" "F.Mask") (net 4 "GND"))
  (pad "2" smd rect (at 0.8 0 180) (size 0.8 0.8) (layers "F.Cu" "F.Paste" "F.Mask") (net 3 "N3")))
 (gr_arc (start 128.171573 81) (mid 127 83.828427) (end 124.171573 85) (stroke (width 0.1) (type default)) (layer "Edge.Cuts"))
 (gr_arc (start 124.171573 64.828427) (mid 127 66) (end 128.171573 68.828427) (stroke (width 0.1) (type default)) (layer "Edge.Cuts"))
 (gr_line (start 110.828427 64.828427) (end 124.171573 64.828427) (stroke (width 0.1) (type default)) (layer "Edge.Cuts"))
 (gr_line (start 106.828427 68.828427) (end 106.828427 81.171573) (stroke (width 0.1) (type default)) (layer "Edge.Cuts"))
 (gr_arc (start 106.828427 68.828427) (mid 108 66) (end 110.828427 64.828427) (stroke (width 0.1) (type default)) (layer "Edge.Cuts"))
 (gr_line (start 128.171573 68.828427) (end 128.171573 81) (stroke (width 0.1) (type default)) (layer "Edge.Cuts"))
 (gr_line (start 124.171573 85) (end 110.828427 85.171573) (stroke (width 0.1) (type default)) (layer "Edge.Cuts"))
 (gr_arc (start 110.828427 85.171573) (mid 108 84) (end 106.828427 81.171573) (stroke (width 0.1) (type default)) (layer "Edge.Cuts"))
 (segment (start 115.5 74) (end 114.5 74) (width 0.25) (layer "F.Cu") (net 4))
 (segment (start 114.5 74) (end 114.1 74.4) (width 0.25) (layer "F.Cu") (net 4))
 (via (at 114.1 74.4) (size 0.8) (drill 0.4) (layers "F.Cu" "B.Cu") (free yes) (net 4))
 (segment (start 111.46 80) (end 108.7 80) (width 0.25) (layer "B.Cu") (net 4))
 (segment (start 113 75.5) (end 108.7 75.5) (width 0.25) (layer "B.Cu") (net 4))
 (segment (start 108.7 75.5) (end 108.7 80) (width 0.25) (layer "B.Cu") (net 4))
 (segment (start 114.1 74.4) (end 113 75.5) (width 0.25) (layer "B.Cu") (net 4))
 (segment (start 117.1 72.3) (end 117.1 74) (width 0.25) (layer "F.Cu") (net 3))
 (segment (start 118 71.4) (end 117.1 72.3) (width 0.25) (layer "F.Cu") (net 3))
 (segment (start 118 70.5) (end 118 71.4) (width 0.25) (layer "F.Cu") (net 3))
 (segment (start 116.5 75.4) (end 116.595 75.305) (width 0.25) (layer "F.Cu") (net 1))
 (segment (start 116.595 75.305) (end 122.5 75.305) (width 0.25) (layer "F.Cu") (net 1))
 (segment (start 116.5 78.8) (end 116.5 75.4) (width 0.25) (layer "F.Cu") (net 1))
 (segment (start 115.3 80) (end 116.5 78.8) (width 0.25) (layer "F.Cu") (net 1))
 (segment (start 114 80) (end 115.3 80) (width 0.25) (layer "F.Cu") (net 1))
 (segment (start 117 68.8) (end 117 67.2) (width 0.25) (layer "F.Cu") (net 2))
 (segment (start 117.605 66.695) (end 122.5 66.695) (width 0.25) (layer "F.Cu") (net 2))
 (segment (start 116.175 70.5) (end 116.175 69.625) (width 0.25) (layer "F.Cu") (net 2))
 (segment (start 117.4 66.8) (end 117.5 66.8) (width 0.25) (layer "F.Cu") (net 2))
 (segment (start 116.175 69.625) (end 117 68.8) (width 0.25) (layer "F.Cu") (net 2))
 (segment (start 117 67.2) (end 117.4 66.8) (width 0.25) (layer "F.Cu") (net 2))
 (segment (start 117.5 66.8) (end 117.605 66.695) (width 0.25) (layer "F.Cu") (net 2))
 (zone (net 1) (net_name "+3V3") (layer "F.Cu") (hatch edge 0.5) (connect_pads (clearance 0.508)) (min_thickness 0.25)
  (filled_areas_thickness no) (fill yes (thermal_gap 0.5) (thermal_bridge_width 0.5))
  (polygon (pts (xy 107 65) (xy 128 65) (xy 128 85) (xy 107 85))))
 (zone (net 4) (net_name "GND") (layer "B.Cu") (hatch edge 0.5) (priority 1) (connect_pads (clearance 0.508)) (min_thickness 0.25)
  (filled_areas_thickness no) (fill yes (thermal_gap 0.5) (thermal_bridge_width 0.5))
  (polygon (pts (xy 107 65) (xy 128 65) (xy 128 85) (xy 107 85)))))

